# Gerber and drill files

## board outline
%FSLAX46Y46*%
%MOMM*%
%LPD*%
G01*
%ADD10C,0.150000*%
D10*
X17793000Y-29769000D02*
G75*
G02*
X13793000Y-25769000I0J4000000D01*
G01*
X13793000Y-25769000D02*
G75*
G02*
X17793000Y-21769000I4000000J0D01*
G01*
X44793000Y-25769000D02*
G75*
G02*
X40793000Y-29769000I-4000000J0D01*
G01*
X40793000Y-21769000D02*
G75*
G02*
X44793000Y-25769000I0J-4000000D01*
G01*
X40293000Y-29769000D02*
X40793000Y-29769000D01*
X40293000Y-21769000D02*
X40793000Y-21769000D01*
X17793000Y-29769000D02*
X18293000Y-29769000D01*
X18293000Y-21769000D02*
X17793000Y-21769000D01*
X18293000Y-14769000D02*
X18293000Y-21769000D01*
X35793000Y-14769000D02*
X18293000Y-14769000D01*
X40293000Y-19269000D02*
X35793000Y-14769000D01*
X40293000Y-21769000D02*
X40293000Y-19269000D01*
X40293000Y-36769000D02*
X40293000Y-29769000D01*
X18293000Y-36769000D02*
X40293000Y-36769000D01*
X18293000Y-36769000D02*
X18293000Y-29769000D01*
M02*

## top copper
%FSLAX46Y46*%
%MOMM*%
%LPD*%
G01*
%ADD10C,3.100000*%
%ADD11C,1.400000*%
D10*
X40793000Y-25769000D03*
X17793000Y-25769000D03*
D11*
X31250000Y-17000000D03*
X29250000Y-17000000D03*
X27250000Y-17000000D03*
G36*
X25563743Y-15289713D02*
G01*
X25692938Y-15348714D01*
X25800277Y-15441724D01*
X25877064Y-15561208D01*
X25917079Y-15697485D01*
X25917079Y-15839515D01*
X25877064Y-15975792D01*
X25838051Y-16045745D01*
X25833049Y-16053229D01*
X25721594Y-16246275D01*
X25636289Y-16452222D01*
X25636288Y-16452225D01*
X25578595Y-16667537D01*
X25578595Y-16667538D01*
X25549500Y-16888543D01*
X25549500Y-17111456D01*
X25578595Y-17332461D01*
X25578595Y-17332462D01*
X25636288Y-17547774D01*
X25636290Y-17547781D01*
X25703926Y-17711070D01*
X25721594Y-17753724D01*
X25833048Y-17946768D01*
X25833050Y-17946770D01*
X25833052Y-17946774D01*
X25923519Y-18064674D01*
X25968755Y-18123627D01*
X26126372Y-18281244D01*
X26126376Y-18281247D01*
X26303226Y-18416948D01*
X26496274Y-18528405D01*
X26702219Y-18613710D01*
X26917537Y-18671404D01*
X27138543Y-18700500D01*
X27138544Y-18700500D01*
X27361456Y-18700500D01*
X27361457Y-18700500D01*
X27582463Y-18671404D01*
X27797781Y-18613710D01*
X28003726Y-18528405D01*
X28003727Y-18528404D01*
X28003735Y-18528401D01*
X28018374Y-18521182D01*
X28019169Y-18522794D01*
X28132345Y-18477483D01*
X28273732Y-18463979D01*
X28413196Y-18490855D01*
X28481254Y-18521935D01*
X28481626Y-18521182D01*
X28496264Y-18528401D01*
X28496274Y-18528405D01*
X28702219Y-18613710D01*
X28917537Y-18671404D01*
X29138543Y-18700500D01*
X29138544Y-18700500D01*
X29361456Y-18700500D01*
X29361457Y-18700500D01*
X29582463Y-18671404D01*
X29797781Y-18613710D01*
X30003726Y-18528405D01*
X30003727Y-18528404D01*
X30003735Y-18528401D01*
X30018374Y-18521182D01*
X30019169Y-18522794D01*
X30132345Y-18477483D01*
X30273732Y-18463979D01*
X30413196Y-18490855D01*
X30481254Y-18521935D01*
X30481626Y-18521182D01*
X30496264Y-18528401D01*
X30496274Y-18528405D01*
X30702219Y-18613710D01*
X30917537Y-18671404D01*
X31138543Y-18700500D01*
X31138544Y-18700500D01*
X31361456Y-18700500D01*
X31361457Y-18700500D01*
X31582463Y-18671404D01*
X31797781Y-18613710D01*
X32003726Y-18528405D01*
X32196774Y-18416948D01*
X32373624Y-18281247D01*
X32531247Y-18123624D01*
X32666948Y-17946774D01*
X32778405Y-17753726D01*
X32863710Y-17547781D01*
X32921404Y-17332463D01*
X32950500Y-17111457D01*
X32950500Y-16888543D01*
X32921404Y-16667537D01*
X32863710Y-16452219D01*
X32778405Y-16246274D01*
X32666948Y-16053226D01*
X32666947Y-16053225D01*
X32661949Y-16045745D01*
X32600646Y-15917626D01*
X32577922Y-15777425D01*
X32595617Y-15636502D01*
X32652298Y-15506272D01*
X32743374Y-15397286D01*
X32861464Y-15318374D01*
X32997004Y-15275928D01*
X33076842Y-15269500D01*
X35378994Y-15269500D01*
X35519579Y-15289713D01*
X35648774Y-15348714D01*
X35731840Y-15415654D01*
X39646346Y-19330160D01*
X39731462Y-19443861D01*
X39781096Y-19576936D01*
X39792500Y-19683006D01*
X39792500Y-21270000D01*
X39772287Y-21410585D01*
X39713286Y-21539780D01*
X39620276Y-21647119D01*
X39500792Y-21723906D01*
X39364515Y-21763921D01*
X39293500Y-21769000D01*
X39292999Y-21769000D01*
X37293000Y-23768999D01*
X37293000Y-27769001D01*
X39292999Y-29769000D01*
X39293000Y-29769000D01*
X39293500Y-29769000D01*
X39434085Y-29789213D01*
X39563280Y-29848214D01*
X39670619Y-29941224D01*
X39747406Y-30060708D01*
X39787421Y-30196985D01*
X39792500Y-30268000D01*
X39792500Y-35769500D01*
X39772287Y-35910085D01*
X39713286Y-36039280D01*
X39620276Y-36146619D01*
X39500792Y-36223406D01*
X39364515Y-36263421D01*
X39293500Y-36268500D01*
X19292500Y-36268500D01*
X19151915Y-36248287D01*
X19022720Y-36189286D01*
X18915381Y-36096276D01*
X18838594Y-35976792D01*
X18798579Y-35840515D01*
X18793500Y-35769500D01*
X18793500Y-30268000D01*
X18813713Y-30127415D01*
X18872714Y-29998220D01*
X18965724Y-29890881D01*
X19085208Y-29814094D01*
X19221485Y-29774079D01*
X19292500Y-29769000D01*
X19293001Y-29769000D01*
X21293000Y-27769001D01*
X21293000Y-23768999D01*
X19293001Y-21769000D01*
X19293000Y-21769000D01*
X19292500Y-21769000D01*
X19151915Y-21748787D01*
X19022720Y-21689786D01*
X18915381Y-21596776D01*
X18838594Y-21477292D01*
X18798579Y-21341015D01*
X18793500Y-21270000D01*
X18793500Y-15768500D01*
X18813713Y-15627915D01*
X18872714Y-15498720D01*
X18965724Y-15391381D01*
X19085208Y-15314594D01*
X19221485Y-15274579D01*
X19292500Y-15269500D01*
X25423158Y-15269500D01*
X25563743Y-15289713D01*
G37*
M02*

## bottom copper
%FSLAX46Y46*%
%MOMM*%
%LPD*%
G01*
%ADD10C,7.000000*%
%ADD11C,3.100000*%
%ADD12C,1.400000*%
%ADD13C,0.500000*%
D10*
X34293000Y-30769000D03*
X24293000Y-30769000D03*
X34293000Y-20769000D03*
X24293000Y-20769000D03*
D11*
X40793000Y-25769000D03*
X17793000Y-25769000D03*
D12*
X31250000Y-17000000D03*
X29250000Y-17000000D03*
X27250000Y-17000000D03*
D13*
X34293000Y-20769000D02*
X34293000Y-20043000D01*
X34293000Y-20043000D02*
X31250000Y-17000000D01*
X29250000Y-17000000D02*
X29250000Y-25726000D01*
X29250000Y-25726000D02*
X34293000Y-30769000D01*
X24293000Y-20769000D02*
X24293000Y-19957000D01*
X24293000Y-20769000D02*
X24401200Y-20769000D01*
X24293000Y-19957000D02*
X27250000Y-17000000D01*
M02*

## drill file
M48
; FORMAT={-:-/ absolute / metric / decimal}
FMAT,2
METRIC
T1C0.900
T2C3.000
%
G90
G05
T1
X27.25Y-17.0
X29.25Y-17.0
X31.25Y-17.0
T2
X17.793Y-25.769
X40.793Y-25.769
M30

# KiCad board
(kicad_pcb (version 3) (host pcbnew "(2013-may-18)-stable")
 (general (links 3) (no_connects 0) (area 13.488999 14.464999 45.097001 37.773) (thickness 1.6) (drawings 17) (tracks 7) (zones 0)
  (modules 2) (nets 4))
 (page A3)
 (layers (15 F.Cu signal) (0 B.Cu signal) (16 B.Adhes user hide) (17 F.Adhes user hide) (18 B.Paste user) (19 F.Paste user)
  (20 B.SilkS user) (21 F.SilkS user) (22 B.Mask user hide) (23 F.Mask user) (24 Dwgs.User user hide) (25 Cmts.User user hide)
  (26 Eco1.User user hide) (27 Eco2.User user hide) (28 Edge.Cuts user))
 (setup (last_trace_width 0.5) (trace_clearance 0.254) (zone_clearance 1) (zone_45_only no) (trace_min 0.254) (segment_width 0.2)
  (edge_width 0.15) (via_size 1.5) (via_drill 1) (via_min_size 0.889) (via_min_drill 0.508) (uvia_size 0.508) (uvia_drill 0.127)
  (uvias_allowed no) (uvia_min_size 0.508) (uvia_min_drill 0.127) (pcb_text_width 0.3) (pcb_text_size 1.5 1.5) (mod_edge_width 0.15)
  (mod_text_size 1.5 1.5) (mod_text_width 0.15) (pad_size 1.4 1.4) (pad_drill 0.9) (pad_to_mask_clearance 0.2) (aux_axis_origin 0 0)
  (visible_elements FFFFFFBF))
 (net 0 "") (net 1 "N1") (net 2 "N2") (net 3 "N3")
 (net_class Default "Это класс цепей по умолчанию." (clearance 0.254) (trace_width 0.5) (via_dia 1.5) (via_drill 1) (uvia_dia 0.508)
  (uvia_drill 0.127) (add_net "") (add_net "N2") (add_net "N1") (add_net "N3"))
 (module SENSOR (layer B.Cu) (at 40.793 37.269 180)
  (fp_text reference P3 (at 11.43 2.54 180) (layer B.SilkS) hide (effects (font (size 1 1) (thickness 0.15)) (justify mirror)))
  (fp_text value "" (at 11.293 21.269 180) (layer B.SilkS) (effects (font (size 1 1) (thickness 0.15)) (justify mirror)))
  (pad 2 smd circle (at 6.5 6.5 180) (size 7 7) (layers B.Cu B.Mask) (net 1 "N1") (solder_mask_margin 0.1))
  (pad 3 smd circle (at 16.5 6.5 180) (size 7 7) (layers B.Cu B.Mask))
  (pad 1 smd circle (at 6.5 16.5 180) (size 7 7) (layers B.Cu B.Mask) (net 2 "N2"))
  (pad 4 smd circle (at 16.5 16.5 180) (size 7 7) (layers B.Cu B.Mask) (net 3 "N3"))
  (pad "" np_thru_hole circle (at 0 11.5 180) (size 3.1 3.1) (drill 3) (layers *.Cu *.Mask B.SilkS))
  (pad "" np_thru_hole circle (at 23 11.5 180) (size 3.1 3.1) (drill 3) (layers *.Cu *.Mask B.SilkS)))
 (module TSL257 (layer F.Cu) (at 29.25 17 180)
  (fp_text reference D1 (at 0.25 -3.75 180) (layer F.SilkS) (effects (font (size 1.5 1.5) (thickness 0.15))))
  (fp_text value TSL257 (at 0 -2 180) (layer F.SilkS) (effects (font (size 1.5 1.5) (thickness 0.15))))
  (pad 1 thru_hole circle (at -2 0 180) (size 1.4 1.4) (drill 0.9) (layers *.Cu *.Mask F.SilkS) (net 2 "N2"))
  (pad 2 thru_hole circle (at 0 0 180) (size 1.4 1.4) (drill 0.9) (layers *.Cu *.Mask F.SilkS) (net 1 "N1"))
  (pad 3 thru_hole circle (at 2 0 180) (size 1.4 1.4) (drill 0.9) (layers *.Cu *.Mask F.SilkS) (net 3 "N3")))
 (gr_arc (start 17.793 25.769) (end 17.793 29.769) (angle 90) (layer Edge.Cuts) (width 0.15))
 (gr_arc (start 17.793 25.769) (end 13.793 25.769) (angle 90) (layer Edge.Cuts) (width 0.15))
 (gr_arc (start 40.793 25.769) (end 44.793 25.769) (angle 90) (layer Edge.Cuts) (width 0.15))
 (gr_arc (start 40.793 25.769) (end 40.793 21.769) (angle 90) (layer Edge.Cuts) (width 0.15))
 (gr_line (start 40.293 29.769) (end 40.793 29.769) (angle 90) (layer Edge.Cuts) (width 0.15))
 (gr_line (start 40.293 21.769) (end 40.793 21.769) (angle 90) (layer Edge.Cuts) (width 0.15))
 (gr_line (start 17.793 29.769) (end 18.293 29.769) (angle 90) (layer Edge.Cuts) (width 0.15))
 (gr_line (start 18.293 21.769) (end 17.793 21.769) (angle 90) (layer Edge.Cuts) (width 0.15))
 (gr_line (start 18.293 14.769) (end 18.293 21.769) (angle 90) (layer Edge.Cuts) (width 0.15))
 (gr_line (start 35.793 14.769) (end 18.293 14.769) (angle 90) (layer Edge.Cuts) (width 0.15))
 (gr_line (start 40.293 19.269) (end 35.793 14.769) (angle 90) (layer Edge.Cuts) (width 0.15))
 (gr_line (start 40.293 21.769) (end 40.293 19.269) (angle 90) (layer Edge.Cuts) (width 0.15))
 (gr_line (start 40.293 36.769) (end 40.293 29.769) (angle 90) (layer Edge.Cuts) (width 0.15))
 (gr_line (start 18.293 36.769) (end 40.293 36.769) (angle 90) (layer Edge.Cuts) (width 0.15))
 (gr_line (start 18.293 36.769) (end 18.293 29.769) (angle 90) (layer Edge.Cuts) (width 0.15))
 (segment (start 34.293 20.769) (end 34.293 20.043) (width 0.5) (layer B.Cu) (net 2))
 (segment (start 34.293 20.043) (end 31.25 17) (width 0.5) (layer B.Cu) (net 2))
 (segment (start 29.25 17) (end 29.25 25.726) (width 0.5) (layer B.Cu) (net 1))
 (segment (start 29.25 25.726) (end 34.293 30.769) (width 0.5) (layer B.Cu) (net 1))
 (segment (start 24.293 20.769) (end 24.293 19.957) (width 0.5) (layer B.Cu) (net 3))
 (segment (start 24.293 20.769) (end 24.4012 20.769) (width 0.5) (layer B.Cu) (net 3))
 (segment (start 24.293 19.957) (end 27.25 17) (width 0.5) (layer B.Cu) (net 3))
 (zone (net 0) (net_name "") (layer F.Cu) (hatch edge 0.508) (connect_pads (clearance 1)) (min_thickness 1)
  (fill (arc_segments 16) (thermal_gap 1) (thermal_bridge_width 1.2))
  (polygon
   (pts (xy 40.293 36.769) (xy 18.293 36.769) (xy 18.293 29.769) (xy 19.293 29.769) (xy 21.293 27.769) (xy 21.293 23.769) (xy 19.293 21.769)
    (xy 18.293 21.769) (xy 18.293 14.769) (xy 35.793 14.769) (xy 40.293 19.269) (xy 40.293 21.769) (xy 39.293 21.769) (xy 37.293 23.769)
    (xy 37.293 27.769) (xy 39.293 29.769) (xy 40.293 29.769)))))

